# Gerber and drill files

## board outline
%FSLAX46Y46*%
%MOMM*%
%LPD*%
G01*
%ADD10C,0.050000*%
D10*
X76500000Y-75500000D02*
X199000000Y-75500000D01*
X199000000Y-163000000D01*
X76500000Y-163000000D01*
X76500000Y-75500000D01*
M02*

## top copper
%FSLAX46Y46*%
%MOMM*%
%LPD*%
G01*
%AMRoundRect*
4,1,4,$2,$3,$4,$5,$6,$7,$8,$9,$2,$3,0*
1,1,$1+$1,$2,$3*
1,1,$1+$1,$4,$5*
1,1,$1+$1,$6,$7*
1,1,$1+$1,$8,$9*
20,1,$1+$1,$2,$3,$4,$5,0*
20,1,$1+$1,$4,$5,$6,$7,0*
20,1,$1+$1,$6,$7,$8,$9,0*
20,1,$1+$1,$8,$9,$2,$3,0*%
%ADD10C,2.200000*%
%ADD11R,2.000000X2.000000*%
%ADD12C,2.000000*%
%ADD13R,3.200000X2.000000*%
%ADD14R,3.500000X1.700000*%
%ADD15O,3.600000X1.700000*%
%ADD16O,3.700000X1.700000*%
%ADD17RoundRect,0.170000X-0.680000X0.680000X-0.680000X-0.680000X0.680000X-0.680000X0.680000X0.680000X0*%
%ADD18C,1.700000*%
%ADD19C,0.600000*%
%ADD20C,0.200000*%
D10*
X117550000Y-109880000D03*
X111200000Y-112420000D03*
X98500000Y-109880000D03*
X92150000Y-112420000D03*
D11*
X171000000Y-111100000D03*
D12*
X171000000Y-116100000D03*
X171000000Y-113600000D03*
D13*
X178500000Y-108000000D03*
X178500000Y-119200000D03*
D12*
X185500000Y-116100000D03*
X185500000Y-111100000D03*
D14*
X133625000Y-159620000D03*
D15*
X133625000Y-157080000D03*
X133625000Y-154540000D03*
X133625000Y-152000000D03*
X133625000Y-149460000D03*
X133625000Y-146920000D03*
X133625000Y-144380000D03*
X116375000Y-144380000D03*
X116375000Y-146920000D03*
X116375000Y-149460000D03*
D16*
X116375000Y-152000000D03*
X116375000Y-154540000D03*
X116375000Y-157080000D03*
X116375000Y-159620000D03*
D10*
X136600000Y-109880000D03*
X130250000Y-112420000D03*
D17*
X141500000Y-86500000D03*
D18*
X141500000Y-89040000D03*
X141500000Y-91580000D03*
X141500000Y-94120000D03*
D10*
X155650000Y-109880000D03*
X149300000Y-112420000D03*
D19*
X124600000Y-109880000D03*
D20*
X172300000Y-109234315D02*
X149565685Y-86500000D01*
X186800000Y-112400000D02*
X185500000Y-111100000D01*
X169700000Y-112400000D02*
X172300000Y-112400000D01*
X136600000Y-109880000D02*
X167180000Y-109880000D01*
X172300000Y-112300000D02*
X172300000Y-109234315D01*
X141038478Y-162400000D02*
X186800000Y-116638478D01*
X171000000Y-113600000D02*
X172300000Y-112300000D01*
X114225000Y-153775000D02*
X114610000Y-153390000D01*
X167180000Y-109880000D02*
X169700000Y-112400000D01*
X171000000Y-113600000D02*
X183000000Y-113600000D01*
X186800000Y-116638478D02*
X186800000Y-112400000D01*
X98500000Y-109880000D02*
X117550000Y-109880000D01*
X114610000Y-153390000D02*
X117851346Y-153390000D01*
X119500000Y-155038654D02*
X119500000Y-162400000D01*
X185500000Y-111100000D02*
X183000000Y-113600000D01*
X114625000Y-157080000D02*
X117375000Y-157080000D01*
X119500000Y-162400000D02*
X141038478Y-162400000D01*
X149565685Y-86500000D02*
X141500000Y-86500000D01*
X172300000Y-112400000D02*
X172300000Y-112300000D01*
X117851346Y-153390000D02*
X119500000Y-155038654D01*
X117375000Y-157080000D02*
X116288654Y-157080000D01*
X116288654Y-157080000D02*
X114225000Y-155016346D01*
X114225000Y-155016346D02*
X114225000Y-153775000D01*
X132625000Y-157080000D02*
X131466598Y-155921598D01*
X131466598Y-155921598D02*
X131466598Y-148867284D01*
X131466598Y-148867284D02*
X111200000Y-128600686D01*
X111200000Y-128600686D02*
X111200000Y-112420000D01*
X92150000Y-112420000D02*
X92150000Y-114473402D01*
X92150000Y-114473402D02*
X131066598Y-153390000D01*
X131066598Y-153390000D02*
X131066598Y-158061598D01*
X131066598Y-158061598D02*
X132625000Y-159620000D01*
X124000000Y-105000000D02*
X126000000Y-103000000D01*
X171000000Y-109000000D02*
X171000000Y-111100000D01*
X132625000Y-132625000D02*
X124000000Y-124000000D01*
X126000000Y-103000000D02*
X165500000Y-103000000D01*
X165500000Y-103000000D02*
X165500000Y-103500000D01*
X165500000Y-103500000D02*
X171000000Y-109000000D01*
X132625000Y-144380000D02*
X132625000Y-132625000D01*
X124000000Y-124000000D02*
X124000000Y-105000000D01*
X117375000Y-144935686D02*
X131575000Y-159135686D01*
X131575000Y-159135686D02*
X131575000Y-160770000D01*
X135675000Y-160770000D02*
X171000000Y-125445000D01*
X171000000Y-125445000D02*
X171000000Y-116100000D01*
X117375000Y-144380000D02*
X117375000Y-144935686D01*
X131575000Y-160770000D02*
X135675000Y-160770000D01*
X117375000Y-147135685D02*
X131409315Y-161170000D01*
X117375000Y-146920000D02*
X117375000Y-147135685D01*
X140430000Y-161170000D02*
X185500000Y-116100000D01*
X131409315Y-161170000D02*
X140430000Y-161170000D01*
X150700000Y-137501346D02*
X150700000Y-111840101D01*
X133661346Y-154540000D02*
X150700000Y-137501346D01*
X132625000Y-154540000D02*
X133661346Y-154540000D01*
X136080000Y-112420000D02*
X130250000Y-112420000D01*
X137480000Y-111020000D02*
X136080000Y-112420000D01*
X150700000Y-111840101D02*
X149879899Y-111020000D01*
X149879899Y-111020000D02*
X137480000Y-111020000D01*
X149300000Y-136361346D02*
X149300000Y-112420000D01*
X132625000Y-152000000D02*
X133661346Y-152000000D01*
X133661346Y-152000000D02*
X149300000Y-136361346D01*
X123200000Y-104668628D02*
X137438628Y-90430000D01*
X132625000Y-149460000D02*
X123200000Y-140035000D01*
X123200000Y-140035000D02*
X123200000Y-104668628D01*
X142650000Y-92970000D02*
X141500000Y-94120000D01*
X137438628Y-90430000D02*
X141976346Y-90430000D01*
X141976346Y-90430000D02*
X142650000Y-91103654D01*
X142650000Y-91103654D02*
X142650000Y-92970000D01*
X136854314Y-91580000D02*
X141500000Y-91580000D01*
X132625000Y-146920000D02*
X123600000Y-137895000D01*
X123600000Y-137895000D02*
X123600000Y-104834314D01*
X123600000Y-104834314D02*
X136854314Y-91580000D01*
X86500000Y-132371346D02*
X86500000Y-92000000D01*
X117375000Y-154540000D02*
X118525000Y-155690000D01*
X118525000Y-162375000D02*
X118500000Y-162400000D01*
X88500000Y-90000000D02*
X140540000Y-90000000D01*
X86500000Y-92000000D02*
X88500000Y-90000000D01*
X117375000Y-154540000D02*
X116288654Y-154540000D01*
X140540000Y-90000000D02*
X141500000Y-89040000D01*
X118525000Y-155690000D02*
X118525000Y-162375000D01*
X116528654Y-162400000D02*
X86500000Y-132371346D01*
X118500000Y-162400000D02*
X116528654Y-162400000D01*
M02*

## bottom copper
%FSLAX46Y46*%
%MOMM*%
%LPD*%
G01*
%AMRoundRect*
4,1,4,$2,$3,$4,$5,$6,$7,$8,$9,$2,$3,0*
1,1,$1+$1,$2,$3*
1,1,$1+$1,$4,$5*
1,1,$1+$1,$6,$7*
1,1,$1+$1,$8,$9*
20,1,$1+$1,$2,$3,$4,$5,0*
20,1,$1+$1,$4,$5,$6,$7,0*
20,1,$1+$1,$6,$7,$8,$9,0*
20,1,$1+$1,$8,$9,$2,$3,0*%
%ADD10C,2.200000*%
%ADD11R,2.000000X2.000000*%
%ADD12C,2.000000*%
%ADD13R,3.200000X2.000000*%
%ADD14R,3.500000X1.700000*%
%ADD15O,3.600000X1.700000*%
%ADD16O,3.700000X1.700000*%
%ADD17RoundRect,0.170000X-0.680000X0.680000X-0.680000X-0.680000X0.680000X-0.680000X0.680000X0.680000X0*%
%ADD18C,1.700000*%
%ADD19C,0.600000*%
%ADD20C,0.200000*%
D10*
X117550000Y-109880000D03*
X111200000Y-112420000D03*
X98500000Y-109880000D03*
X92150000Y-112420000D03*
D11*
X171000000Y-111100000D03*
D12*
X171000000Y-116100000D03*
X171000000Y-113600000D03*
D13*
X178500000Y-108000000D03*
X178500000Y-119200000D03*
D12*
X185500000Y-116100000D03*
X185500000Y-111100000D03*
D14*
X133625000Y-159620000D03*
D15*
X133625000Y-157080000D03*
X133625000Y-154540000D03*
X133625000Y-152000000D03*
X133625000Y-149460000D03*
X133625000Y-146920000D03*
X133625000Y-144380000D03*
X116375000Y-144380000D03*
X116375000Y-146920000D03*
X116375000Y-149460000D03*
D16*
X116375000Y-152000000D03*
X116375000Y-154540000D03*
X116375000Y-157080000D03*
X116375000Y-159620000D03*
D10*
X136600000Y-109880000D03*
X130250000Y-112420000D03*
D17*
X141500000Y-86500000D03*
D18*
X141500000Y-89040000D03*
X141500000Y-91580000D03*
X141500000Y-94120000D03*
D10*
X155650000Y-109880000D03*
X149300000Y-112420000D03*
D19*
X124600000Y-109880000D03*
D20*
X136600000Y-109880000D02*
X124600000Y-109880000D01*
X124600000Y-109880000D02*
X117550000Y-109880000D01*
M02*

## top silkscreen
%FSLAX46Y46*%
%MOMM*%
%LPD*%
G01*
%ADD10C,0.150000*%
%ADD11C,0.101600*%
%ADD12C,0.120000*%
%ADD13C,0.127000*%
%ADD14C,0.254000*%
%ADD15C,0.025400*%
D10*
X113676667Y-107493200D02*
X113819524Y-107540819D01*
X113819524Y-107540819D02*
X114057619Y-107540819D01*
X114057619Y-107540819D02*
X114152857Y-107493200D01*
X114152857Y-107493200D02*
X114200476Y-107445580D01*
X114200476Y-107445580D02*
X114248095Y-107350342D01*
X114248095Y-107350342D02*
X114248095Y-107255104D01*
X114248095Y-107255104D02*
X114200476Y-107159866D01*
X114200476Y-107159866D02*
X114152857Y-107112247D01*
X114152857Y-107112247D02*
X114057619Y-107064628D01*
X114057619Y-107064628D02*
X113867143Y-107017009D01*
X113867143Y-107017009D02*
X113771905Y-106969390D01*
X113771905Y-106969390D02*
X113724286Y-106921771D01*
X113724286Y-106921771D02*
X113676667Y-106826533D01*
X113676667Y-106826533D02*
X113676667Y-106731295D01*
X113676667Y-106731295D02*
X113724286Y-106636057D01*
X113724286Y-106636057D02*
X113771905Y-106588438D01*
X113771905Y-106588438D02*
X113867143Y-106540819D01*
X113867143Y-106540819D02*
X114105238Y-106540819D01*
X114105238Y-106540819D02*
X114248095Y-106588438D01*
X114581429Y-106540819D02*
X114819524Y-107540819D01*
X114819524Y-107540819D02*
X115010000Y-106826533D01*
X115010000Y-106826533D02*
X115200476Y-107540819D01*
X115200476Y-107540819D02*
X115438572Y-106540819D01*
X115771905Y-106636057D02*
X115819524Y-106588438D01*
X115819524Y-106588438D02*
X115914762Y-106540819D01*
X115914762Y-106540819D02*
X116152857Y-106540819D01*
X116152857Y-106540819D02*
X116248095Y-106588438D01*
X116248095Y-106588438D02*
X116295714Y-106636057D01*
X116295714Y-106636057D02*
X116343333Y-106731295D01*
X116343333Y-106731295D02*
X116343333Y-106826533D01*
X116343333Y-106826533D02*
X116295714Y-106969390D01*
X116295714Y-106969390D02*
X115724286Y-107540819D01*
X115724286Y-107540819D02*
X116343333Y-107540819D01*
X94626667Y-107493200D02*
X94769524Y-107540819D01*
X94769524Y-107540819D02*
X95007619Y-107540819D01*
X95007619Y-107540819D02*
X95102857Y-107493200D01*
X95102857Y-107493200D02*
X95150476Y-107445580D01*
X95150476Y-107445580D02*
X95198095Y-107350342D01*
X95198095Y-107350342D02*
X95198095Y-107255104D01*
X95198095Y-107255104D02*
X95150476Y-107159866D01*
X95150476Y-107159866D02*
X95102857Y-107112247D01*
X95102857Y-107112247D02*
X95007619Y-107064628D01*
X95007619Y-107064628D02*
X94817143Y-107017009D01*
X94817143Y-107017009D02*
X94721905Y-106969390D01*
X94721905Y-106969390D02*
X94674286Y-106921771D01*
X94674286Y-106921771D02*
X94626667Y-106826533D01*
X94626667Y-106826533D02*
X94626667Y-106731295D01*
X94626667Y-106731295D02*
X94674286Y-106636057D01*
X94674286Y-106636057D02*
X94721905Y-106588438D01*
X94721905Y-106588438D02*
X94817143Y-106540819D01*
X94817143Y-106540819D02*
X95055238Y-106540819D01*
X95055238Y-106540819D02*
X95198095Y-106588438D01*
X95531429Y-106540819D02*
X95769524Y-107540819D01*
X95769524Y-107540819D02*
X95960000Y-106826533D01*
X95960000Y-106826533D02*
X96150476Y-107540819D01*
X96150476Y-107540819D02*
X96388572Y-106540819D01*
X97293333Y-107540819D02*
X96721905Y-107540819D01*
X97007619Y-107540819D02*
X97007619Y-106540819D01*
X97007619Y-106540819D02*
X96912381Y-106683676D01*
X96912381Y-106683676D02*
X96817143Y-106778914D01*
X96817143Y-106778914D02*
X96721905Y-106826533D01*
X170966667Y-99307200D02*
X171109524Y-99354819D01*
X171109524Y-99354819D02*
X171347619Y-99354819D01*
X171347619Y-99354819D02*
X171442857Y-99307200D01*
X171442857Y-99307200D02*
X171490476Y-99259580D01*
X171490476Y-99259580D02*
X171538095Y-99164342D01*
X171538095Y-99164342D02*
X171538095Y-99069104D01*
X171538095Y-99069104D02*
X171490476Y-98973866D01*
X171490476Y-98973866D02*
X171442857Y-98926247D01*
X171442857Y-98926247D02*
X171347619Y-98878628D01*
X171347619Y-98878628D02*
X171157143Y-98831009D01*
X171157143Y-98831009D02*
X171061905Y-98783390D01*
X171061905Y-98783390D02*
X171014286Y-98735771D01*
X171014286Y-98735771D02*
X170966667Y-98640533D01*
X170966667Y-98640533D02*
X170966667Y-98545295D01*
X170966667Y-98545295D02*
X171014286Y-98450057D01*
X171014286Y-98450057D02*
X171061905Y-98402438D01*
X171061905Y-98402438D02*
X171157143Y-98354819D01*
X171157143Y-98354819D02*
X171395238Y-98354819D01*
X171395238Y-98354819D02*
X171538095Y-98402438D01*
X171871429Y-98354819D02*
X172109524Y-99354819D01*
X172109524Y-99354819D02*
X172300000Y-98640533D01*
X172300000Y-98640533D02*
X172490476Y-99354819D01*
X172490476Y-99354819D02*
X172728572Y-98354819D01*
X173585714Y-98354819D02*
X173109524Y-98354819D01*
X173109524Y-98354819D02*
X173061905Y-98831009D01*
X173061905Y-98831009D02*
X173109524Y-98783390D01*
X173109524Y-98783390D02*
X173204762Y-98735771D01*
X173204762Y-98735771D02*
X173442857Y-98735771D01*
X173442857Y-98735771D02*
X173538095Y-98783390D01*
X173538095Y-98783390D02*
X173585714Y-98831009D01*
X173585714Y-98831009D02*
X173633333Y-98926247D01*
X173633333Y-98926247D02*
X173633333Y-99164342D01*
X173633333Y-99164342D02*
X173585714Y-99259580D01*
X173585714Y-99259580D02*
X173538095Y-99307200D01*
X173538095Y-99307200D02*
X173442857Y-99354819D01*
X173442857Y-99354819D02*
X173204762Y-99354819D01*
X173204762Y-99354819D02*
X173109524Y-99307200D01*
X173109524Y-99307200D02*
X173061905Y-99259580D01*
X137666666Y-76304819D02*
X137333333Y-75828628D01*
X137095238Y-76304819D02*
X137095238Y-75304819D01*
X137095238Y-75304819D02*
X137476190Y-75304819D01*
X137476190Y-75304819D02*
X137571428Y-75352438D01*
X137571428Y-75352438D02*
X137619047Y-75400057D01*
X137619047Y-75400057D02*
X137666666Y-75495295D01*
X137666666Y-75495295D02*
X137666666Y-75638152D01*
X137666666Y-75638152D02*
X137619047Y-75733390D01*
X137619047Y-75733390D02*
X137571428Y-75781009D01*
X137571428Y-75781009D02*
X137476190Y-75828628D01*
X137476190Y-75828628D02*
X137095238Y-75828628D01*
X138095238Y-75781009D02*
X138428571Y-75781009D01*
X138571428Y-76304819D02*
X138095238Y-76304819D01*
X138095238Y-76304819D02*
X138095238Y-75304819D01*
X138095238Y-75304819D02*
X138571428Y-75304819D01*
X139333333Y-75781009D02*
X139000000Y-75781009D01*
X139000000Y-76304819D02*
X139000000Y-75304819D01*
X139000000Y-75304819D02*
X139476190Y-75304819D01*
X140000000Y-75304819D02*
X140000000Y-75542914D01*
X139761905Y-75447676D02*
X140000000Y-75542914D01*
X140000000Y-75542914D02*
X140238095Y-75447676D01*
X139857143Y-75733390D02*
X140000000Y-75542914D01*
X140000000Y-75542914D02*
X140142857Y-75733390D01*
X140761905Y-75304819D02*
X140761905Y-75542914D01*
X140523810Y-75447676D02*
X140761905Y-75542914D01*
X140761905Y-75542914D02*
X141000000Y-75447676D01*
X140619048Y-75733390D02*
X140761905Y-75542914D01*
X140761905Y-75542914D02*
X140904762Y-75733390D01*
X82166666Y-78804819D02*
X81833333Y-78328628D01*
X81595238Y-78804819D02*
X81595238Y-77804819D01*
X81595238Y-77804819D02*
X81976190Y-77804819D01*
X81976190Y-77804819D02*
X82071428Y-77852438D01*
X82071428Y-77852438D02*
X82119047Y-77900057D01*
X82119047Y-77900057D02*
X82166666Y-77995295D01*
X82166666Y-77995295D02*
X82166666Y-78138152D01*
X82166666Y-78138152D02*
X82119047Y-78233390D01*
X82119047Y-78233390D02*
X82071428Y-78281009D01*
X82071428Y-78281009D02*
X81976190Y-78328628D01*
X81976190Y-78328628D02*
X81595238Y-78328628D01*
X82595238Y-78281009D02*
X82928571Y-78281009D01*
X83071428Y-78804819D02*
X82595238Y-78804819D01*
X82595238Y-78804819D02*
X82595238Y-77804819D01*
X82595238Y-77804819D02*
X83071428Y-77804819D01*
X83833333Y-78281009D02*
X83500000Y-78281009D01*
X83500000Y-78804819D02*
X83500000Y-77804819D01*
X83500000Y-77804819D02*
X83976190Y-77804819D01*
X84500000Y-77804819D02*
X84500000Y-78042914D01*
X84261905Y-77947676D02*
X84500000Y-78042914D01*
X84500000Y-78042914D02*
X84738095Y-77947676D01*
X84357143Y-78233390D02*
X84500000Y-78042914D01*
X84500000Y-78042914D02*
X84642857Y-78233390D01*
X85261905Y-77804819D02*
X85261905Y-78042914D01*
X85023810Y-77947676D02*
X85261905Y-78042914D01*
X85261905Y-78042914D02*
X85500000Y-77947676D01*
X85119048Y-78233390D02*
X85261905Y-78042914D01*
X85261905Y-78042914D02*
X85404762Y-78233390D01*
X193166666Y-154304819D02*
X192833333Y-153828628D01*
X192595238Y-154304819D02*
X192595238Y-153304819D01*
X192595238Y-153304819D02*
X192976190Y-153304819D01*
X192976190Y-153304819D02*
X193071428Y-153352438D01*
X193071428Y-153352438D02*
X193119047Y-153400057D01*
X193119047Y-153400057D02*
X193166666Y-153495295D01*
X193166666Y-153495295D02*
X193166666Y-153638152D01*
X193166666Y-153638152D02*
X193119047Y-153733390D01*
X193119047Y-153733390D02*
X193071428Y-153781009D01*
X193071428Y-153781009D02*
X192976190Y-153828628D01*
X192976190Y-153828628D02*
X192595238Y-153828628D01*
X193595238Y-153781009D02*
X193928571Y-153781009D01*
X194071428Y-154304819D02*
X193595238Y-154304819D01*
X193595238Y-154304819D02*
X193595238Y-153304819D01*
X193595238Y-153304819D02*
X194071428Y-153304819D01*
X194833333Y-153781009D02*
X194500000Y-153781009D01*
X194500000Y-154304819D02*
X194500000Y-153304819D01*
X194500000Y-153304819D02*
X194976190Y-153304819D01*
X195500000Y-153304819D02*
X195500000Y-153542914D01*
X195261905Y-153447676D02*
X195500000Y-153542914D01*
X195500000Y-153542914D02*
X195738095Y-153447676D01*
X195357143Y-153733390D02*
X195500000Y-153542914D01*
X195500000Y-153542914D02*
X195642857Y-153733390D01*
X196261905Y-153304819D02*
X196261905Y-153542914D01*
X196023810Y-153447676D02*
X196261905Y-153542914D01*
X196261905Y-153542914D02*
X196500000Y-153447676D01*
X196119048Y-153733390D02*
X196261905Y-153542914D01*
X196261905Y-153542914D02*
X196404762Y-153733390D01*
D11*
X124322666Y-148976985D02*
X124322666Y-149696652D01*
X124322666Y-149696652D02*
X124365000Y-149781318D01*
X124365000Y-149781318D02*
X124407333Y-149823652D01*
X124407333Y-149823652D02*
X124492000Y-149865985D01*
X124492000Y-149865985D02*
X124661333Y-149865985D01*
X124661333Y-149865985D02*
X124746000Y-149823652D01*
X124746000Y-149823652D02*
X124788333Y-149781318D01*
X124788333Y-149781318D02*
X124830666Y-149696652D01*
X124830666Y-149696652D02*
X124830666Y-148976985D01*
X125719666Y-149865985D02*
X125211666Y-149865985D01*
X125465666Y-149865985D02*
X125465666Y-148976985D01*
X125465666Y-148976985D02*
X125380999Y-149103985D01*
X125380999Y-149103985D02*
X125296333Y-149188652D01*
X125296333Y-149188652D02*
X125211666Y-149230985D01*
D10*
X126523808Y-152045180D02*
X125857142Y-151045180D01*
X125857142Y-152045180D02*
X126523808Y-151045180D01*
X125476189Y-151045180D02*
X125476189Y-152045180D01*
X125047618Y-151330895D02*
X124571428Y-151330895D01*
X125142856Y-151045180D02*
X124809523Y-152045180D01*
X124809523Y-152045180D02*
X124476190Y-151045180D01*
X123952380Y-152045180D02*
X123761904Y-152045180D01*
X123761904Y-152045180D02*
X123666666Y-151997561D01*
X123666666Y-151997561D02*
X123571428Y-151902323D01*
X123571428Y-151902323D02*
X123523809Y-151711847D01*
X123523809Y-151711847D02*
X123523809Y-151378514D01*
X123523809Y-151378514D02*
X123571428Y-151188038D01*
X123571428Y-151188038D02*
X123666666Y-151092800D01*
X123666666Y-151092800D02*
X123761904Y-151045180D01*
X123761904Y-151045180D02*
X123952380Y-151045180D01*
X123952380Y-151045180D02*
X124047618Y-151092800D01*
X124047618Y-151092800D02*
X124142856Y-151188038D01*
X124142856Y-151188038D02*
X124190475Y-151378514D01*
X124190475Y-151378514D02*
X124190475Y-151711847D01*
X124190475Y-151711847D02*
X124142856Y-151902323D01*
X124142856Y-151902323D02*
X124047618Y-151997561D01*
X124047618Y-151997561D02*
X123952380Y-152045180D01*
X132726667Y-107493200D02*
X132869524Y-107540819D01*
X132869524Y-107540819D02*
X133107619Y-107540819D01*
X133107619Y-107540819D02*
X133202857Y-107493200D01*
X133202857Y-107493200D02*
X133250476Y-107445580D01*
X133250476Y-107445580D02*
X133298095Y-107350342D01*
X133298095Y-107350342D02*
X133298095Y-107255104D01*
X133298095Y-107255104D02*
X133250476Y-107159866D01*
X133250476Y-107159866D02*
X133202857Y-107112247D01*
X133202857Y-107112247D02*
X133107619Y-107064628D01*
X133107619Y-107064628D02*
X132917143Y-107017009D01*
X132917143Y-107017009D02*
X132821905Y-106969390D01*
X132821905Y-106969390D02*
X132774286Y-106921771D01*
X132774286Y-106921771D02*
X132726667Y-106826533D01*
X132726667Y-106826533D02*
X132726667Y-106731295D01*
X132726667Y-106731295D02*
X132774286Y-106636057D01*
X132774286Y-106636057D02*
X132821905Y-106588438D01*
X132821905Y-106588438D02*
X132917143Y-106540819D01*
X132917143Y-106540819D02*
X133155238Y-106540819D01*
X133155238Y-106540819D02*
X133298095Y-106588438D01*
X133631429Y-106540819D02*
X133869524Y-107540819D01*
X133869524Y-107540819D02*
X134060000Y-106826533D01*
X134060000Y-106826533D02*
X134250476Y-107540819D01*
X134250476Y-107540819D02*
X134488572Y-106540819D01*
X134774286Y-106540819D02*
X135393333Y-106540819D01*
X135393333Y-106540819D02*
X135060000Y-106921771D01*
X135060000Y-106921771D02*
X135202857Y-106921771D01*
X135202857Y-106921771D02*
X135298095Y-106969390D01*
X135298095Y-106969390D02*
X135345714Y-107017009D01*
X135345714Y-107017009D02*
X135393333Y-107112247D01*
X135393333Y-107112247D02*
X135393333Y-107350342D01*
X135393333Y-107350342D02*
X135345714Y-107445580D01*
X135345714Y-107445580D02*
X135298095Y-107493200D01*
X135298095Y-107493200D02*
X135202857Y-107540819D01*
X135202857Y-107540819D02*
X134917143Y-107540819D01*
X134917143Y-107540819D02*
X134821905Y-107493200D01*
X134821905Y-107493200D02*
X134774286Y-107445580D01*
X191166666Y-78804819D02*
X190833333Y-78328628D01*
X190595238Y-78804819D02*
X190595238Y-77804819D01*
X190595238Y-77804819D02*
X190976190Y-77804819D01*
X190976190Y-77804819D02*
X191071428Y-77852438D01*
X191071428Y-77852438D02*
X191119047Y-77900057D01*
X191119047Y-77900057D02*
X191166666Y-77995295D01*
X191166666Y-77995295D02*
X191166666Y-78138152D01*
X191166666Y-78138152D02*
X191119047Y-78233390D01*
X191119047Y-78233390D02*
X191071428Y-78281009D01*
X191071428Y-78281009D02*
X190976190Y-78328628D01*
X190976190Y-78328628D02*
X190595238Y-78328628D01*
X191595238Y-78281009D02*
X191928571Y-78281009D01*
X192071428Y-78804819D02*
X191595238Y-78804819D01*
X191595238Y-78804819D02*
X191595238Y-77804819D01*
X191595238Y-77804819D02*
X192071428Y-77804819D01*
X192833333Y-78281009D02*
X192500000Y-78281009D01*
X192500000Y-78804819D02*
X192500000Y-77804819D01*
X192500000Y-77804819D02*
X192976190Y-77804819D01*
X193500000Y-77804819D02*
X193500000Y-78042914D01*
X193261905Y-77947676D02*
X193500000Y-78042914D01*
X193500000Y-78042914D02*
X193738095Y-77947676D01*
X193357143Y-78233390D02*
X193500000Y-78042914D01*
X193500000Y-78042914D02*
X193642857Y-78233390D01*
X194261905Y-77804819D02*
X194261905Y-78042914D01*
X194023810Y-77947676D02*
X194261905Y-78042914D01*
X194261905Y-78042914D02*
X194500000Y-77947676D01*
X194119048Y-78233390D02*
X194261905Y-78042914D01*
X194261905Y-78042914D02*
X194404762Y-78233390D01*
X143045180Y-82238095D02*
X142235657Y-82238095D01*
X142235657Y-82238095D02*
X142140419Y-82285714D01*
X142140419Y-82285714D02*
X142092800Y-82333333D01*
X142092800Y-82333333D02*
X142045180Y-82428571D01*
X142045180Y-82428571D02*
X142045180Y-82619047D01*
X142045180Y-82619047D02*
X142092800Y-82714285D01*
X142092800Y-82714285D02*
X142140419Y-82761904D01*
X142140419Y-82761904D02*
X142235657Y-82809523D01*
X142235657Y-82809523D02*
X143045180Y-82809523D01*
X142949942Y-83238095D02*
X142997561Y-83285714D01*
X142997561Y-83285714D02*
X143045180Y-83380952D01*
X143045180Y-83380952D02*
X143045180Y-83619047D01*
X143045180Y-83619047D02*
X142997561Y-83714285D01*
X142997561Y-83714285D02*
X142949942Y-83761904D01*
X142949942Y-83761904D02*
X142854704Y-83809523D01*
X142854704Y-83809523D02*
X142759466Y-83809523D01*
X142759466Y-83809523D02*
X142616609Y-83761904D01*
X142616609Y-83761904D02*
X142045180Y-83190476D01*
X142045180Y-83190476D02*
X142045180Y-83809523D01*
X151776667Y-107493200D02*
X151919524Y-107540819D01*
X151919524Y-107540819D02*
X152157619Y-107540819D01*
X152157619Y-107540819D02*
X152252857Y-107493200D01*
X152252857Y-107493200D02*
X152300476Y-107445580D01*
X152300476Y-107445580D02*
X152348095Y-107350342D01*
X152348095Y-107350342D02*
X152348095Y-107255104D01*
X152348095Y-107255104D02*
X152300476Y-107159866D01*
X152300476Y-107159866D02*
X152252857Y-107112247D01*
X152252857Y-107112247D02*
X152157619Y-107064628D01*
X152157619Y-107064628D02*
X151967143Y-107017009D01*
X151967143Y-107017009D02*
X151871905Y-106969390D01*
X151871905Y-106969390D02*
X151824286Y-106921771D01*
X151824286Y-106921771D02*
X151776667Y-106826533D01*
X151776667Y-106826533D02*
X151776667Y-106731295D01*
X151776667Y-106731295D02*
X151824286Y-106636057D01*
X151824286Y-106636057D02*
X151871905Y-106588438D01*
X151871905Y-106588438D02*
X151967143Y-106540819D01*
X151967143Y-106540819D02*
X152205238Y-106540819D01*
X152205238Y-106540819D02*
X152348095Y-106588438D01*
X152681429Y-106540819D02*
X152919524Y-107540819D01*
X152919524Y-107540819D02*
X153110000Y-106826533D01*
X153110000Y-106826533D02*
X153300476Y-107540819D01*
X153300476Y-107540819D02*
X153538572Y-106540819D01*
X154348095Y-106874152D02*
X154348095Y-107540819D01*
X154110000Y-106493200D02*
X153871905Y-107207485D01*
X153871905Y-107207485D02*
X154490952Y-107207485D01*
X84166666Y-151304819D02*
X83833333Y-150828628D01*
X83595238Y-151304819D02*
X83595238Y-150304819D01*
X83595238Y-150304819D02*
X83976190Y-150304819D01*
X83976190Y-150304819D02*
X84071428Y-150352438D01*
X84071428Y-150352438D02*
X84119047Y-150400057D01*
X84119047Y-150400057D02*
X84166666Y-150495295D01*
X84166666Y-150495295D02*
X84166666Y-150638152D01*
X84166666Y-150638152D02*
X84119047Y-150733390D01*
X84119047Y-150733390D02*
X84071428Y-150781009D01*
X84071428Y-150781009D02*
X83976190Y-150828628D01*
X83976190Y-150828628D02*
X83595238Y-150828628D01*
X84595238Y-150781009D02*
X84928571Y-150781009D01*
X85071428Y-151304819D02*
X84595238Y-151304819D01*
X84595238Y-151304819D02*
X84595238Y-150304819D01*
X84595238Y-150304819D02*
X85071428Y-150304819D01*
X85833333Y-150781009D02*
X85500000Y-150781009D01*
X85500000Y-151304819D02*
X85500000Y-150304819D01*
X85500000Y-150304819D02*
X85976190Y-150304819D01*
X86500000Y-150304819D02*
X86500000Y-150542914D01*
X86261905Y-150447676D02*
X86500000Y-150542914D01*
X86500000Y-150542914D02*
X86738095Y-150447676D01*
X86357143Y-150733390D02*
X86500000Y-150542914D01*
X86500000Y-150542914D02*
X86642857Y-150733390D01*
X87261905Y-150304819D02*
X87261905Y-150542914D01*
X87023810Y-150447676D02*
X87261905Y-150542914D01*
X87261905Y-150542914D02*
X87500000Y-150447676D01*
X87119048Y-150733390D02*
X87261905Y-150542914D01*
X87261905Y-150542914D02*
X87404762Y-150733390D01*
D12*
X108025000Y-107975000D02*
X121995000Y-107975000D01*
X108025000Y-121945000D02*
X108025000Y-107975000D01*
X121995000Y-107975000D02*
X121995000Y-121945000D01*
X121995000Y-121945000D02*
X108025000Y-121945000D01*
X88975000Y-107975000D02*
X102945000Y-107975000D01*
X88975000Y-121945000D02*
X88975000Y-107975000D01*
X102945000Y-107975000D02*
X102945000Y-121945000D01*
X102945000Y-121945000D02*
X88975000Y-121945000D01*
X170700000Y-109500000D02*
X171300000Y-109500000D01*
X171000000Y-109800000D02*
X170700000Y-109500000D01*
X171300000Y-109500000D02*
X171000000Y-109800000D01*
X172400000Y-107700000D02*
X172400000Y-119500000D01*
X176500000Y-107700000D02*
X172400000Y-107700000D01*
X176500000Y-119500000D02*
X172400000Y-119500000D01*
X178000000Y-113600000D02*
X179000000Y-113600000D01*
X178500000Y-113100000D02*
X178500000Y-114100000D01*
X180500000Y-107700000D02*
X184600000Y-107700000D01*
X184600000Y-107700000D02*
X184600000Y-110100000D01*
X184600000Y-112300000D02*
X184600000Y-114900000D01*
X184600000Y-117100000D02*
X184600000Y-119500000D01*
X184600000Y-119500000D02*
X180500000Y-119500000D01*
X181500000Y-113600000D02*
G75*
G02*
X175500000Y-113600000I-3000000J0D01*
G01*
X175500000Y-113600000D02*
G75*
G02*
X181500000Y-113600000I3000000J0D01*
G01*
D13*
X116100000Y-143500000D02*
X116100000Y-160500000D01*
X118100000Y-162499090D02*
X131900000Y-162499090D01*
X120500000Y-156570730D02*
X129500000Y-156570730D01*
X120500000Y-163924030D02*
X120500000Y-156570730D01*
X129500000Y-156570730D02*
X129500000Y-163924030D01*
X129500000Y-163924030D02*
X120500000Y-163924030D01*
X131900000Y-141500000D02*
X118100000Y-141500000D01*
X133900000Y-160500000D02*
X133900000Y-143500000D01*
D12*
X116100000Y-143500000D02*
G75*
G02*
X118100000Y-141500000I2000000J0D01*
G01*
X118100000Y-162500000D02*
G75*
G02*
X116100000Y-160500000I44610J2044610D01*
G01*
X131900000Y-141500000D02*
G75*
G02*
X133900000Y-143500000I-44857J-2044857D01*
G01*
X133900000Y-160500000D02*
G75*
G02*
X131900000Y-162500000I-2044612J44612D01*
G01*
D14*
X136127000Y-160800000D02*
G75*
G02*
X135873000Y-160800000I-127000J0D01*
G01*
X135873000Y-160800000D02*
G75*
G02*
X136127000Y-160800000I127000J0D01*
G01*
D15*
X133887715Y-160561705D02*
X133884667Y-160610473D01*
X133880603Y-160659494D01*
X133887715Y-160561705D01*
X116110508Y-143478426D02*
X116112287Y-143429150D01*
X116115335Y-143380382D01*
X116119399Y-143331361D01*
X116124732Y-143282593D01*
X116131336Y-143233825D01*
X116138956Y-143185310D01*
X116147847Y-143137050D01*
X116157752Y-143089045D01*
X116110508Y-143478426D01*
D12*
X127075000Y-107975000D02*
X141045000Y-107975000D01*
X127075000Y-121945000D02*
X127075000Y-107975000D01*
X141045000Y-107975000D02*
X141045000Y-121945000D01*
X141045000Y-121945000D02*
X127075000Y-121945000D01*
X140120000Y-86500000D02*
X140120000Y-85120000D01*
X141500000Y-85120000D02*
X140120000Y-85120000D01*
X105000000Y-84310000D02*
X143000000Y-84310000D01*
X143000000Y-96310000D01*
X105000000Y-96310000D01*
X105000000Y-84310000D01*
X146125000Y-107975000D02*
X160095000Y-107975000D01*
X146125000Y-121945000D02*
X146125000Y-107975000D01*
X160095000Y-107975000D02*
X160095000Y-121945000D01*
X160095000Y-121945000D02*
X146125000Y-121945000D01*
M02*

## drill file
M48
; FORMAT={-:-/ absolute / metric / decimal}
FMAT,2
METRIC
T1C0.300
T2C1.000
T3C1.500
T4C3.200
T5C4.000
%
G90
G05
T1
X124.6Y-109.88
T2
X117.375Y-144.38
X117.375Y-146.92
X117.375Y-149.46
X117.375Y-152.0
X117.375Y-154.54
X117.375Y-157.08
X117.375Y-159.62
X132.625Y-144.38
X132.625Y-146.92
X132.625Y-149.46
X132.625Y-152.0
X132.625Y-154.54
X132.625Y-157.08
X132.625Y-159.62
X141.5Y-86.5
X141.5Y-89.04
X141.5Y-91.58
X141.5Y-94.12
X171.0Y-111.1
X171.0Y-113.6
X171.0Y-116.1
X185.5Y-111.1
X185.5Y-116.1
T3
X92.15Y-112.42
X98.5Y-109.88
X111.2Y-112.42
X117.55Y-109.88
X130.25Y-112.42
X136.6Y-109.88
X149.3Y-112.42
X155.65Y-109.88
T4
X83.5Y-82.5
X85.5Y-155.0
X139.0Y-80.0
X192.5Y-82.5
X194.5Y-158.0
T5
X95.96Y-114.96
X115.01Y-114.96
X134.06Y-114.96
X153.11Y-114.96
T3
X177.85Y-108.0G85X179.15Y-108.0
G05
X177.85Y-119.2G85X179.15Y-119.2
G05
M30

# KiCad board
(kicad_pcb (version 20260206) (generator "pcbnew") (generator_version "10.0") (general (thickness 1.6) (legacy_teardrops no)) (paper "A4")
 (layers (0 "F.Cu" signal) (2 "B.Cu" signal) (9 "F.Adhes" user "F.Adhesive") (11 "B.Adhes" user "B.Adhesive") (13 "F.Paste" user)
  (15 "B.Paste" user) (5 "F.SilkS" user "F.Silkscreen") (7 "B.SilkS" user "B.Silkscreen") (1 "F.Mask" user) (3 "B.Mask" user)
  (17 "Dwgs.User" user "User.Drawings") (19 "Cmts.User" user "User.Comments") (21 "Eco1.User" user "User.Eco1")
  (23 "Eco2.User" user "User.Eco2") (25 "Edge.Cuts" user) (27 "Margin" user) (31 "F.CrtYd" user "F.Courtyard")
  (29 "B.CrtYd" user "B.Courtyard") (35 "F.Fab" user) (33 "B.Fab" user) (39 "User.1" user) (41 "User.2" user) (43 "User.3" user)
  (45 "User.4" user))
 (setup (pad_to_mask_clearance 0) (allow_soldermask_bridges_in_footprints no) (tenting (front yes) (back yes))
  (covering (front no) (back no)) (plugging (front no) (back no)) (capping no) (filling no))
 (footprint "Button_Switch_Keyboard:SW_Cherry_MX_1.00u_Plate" (layer "F.Cu") (at 117.55 109.88)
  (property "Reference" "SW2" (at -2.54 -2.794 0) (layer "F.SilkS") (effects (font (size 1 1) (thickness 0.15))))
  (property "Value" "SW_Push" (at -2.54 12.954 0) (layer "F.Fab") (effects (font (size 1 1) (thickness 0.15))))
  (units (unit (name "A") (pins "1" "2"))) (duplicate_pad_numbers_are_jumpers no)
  (fp_line (start -9.525 -1.905) (end 4.445 -1.905) (stroke (width 0.12) (type solid)) (layer "F.SilkS"))
  (fp_line (start -9.525 12.065) (end -9.525 -1.905) (stroke (width 0.12) (type solid)) (layer "F.SilkS"))
  (fp_line (start 4.445 -1.905) (end 4.445 12.065) (stroke (width 0.12) (type solid)) (layer "F.SilkS"))
  (fp_line (start 4.445 12.065) (end -9.525 12.065) (stroke (width 0.12) (type solid)) (layer "F.SilkS"))
  (pad "" np_thru_hole circle (at -2.54 5.08) (size 4 4) (drill 4) (layers "*.Cu" "*.Mask"))
  (pad "1" thru_hole circle (at 0 0) (size 2.2 2.2) (drill 1.5) (layers "*.Cu" "*.Mask") (remove_unused_layers no) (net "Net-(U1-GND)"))
  (pad "2" thru_hole circle (at -6.35 2.54) (size 2.2 2.2) (drill 1.5) (layers "*.Cu" "*.Mask") (remove_unused_layers no)
   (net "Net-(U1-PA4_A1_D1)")))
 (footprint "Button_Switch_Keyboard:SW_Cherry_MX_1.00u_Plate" (layer "F.Cu") (at 98.5 109.88)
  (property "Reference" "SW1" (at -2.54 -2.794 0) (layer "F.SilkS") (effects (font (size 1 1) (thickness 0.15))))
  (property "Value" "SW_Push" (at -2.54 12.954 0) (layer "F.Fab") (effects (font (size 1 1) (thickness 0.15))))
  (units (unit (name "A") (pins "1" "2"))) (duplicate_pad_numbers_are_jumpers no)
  (fp_line (start -9.525 -1.905) (end 4.445 -1.905) (stroke (width 0.12) (type solid)) (layer "F.SilkS"))
  (fp_line (start -9.525 12.065) (end -9.525 -1.905) (stroke (width 0.12) (type solid)) (layer "F.SilkS"))
  (fp_line (start 4.445 -1.905) (end 4.445 12.065) (stroke (width 0.12) (type solid)) (layer "F.SilkS"))
  (fp_line (start 4.445 12.065) (end -9.525 12.065) (stroke (width 0.12) (type solid)) (layer "F.SilkS"))
  (pad "" np_thru_hole circle (at -2.54 5.08) (size 4 4) (drill 4) (layers "*.Cu" "*.Mask"))
  (pad "1" thru_hole circle (at 0 0) (size 2.2 2.2) (drill 1.5) (layers "*.Cu" "*.Mask") (remove_unused_layers no) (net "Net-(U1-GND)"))
  (pad "2" thru_hole circle (at -6.35 2.54) (size 2.2 2.2) (drill 1.5) (layers "*.Cu" "*.Mask") (remove_unused_layers no)
   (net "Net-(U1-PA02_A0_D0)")))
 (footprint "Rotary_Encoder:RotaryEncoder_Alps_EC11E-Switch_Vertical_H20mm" (layer "F.Cu") (at 171 111.1)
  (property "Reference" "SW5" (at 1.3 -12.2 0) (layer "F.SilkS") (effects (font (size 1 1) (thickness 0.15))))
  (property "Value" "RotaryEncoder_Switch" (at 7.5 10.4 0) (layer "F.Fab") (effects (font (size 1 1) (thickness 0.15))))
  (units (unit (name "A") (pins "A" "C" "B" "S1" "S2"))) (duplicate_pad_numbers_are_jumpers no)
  (fp_line (start -0.3 -1.6) (end 0.3 -1.6) (stroke (width 0.12) (type solid)) (layer "F.SilkS"))
  (fp_line (start 0 -1.3) (end -0.3 -1.6) (stroke (width 0.12) (type solid)) (layer "F.SilkS"))
  (fp_line (start 0.3 -1.6) (end 0 -1.3) (stroke (width 0.12) (type solid)) (layer "F.SilkS"))
  (fp_line (start 1.4 -3.4) (end 1.4 8.4) (stroke (width 0.12) (type solid)) (layer "F.SilkS"))
  (fp_line (start 5.5 -3.4) (end 1.4 -3.4) (stroke (width 0.12) (type solid)) (layer "F.SilkS"))
  (fp_line (start 5.5 8.4) (end 1.4 8.4) (stroke (width 0.12) (type solid)) (layer "F.SilkS"))
  (fp_line (start 7 2.5) (end 8 2.5) (stroke (width 0.12) (type solid)) (layer "F.SilkS"))
  (fp_line (start 7.5 2) (end 7.5 3) (stroke (width 0.12) (type solid)) (layer "F.SilkS"))
  (fp_line (start 9.5 -3.4) (end 13.6 -3.4) (stroke (width 0.12) (type solid)) (layer "F.SilkS"))
  (fp_line (start 13.6 -3.4) (end 13.6 -1) (stroke (width 0.12) (type solid)) (layer "F.SilkS"))
  (fp_line (start 13.6 1.2) (end 13.6 3.8) (stroke (width 0.12) (type solid)) (layer "F.SilkS"))
  (fp_line (start 13.6 6) (end 13.6 8.4) (stroke (width 0.12) (type solid)) (layer "F.SilkS"))
  (fp_line (start 13.6 8.4) (end 9.5 8.4) (stroke (width 0.12) (type solid)) (layer "F.SilkS"))
  (fp_circle (center 7.5 2.5) (end 10.5 2.5) (stroke (width 0.12) (type solid)) (fill no) (layer "F.SilkS"))
  (pad "A" thru_hole rect (at 0 0) (size 2 2) (drill 1) (layers "*.Cu" "*.Mask") (remove_unused_layers no) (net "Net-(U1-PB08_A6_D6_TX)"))
  (pad "B" thru_hole circle (at 0 5) (size 2 2) (drill 1) (layers "*.Cu" "*.Mask") (remove_unused_layers no) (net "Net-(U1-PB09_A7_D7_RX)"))
  (pad "C" thru_hole circle (at 0 2.5) (size 2 2) (drill 1) (layers "*.Cu" "*.Mask") (remove_unused_layers no) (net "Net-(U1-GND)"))
  (pad "MP" thru_hole rect (at 7.5 -3.1) (size 3.2 2) (drill oval 2.8 1.5) (layers "*.Cu" "*.Mask") (remove_unused_layers no))
  (pad "MP" thru_hole rect (at 7.5 8.1) (size 3.2 2) (drill oval 2.8 1.5) (layers "*.Cu" "*.Mask") (remove_unused_layers no))
  (pad "S1" thru_hole circle (at 14.5 5) (size 2 2) (drill 1) (layers "*.Cu" "*.Mask") (remove_unused_layers no)
   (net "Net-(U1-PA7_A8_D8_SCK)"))
  (pad "S2" thru_hole circle (at 14.5 0) (size 2 2) (drill 1) (layers "*.Cu" "*.Mask") (remove_unused_layers no) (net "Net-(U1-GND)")))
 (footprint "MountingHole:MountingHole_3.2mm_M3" (layer "F.Cu") (at 139 80)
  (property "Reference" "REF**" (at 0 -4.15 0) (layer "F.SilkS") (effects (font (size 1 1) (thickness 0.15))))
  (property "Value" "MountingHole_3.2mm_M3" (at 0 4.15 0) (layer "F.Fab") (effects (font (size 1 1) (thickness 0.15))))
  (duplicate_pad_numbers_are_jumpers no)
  (pad "" np_thru_hole circle (at 0 0) (size 3.2 3.2) (drill 3.2) (layers "*.Cu" "*.Mask")))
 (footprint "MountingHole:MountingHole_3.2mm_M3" (layer "F.Cu") (at 83.5 82.5)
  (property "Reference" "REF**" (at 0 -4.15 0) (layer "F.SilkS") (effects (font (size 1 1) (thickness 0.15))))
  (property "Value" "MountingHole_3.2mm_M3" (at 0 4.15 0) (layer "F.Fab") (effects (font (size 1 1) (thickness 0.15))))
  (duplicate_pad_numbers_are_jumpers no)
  (pad "" np_thru_hole circle (at 0 0) (size 3.2 3.2) (drill 3.2) (layers "*.Cu" "*.Mask")))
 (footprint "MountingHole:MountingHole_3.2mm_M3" (layer "F.Cu") (at 194.5 158)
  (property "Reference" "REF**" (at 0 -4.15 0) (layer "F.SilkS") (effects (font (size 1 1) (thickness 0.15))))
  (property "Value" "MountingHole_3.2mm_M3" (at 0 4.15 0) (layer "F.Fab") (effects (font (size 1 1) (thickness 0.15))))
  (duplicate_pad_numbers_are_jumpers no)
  (pad "" np_thru_hole circle (at 0 0) (size 3.2 3.2) (drill 3.2) (layers "*.Cu" "*.Mask")))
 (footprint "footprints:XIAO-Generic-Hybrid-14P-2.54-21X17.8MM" (layer "F.Cu") (at 125 152 180)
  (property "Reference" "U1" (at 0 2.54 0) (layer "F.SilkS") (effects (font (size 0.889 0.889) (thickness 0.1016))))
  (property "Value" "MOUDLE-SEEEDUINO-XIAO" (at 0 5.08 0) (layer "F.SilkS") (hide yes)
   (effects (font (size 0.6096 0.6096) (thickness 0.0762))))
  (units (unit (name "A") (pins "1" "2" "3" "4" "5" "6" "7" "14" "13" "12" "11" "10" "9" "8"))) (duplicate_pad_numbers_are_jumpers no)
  (fp_line (start 8.9 8.5) (end 8.9 -8.5) (stroke (width 0.127) (type solid)) (layer "F.SilkS"))
  (fp_line (start 6.9 -10.49909) (end -6.9 -10.49909) (stroke (width 0.127) (type solid)) (layer "F.SilkS"))
  (fp_line (start 4.5 -4.57073) (end -4.5 -4.57073) (stroke (width 0.127) (type solid)) (layer "F.SilkS"))
  (fp_line (start 4.5 -11.92403) (end 4.5 -4.57073) (stroke (width 0.127) (type solid)) (layer "F.SilkS"))
  (fp_line (start -4.5 -4.57073) (end -4.5 -11.92403) (stroke (width 0.127) (type solid)) (layer "F.SilkS"))
  (fp_line (start -4.5 -11.92403) (end 4.5 -11.92403) (stroke (width 0.127) (type solid)) (layer "F.SilkS"))
  (fp_line (start -6.9 10.5) (end 6.9 10.5) (stroke (width 0.127) (type solid)) (layer "F.SilkS"))
  (fp_line (start -8.9 -8.5) (end -8.9 8.5) (stroke (width 0.127) (type solid)) (layer "F.SilkS"))
  (fp_arc (start 8.9 8.5) (mid 8.314214 9.914214) (end 6.9 10.5) (stroke (width 0.12) (type solid)) (layer "F.SilkS"))
  (fp_arc (start 6.9 -10.5) (mid 8.301491 -9.901491) (end 8.9 -8.5) (stroke (width 0.12) (type solid)) (layer "F.SilkS"))
  (fp_arc (start -6.9 10.5) (mid -8.301423 9.901423) (end -8.9 8.5) (stroke (width 0.12) (type solid)) (layer "F.SilkS"))
  (fp_arc (start -8.9 -8.5) (mid -8.301491 -9.901491) (end -6.9 -10.5) (stroke (width 0.12) (type solid)) (layer "F.SilkS"))
  (fp_circle (center -11 -8.8) (end -11 -9.054) (stroke (width 0) (type solid)) (fill yes) (layer "F.SilkS"))
  (fp_poly
   (pts (xy -8.887715 -8.561705) (xy -8.884667 -8.610473) (xy -8.880603 -8.659494)) (stroke (width 0.0254) (type solid)) (fill no)
   (layer "F.SilkS"))
  (fp_poly
   (pts (xy 8.889492 8.521574) (xy 8.887713 8.57085) (xy 8.884665 8.619618) (xy 8.880601 8.668639) (xy 8.875268 8.717407)
    (xy 8.868664 8.766175) (xy 8.861044 8.81469) (xy 8.852153 8.86295) (xy 8.842248 8.910955))
   (stroke (width 0.0254) (type solid)) (fill no) (layer "F.SilkS"))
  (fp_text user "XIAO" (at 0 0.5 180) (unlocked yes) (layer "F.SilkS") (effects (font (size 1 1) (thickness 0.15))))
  (pad "1" thru_hole rect (at -7.625 -7.62 180) (size 3.5 1.7) (drill 1 (offset -1 0)) (layers "*.Cu" "*.Mask") (remove_unused_layers no)
   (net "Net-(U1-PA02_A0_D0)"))
  (pad "2" thru_hole oval (at -7.625 -5.08 180) (size 3.6 1.7) (drill 1 (offset -1 0)) (layers "*.Cu" "*.Mask") (remove_unused_layers no)
   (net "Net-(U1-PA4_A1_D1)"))
  (pad "3" thru_hole oval (at -7.625 -2.54 180) (size 3.6 1.7) (drill 1 (offset -1 0)) (layers "*.Cu" "*.Mask") (remove_unused_layers no)
   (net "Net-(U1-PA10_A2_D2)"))
  (pad "4" thru_hole oval (at -7.625 0 180) (size 3.6 1.7) (drill 1 (offset -1 0)) (layers "*.Cu" "*.Mask") (remove_unused_layers no)
   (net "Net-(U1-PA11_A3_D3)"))
  (pad "5" thru_hole oval (at -7.625 2.54 180) (size 3.6 1.7) (drill 1 (offset -1 0)) (layers "*.Cu" "*.Mask") (remove_unused_layers no)
   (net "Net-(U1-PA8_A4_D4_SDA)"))
  (pad "6" thru_hole oval (at -7.625 5.08) (size 3.6 1.7) (drill 1 (offset 1 0)) (layers "*.Cu" "*.Mask") (remove_unused_layers no)
   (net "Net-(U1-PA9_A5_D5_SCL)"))
  (pad "7" thru_hole oval (at -7.625 7.62 180) (size 3.6 1.7) (drill 1 (offset -1 0)) (layers "*.Cu" "*.Mask") (remove_unused_layers no)
   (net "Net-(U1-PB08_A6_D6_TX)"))
  (pad "8" thru_hole oval (at 7.625 7.62 180) (size 3.6 1.7) (drill 1 (offset 1 0)) (layers "*.Cu" "*.Mask") (remove_unused_layers no)
   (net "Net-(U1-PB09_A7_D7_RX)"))
  (pad "9" thru_hole oval (at 7.625 5.08 180) (size 3.6 1.7) (drill 1 (offset 1 0)) (layers "*.Cu" "*.Mask") (remove_unused_layers no)
   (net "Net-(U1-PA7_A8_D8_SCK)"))
  (pad "10" thru_hole oval (at 7.625 2.54 180) (size 3.6 1.7) (drill 1 (offset 1 0)) (layers "*.Cu" "*.Mask") (remove_unused_layers no)
   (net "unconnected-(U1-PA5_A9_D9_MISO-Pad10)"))
  (pad "11" thru_hole oval (at 7.625 0 180) (size 3.7 1.7) (drill 1 (offset 1 0)) (layers "*.Cu" "*.Mask") (remove_unused_layers no)
   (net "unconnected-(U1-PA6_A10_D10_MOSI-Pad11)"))
  (pad "12" thru_hole oval (at 7.625 -2.54 180) (size 3.7 1.7) (drill 1 (offset 1 0)) (layers "*.Cu" "*.Mask") (remove_unused_layers no)
   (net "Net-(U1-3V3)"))
  (pad "13" thru_hole oval (at 7.625 -5.08 180) (size 3.7 1.7) (drill 1 (offset 1 0)) (layers "*.Cu" "*.Mask") (remove_unused_layers no)
   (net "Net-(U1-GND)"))
  (pad "14" thru_hole oval (at 7.625 -7.62 180) (size 3.7 1.7) (drill 1 (offset 1 0)) (layers "*.Cu" "*.Mask") (remove_unused_layers no)
   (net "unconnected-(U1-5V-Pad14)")))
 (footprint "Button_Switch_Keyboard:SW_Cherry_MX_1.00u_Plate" (layer "F.Cu") (at 136.6 109.88)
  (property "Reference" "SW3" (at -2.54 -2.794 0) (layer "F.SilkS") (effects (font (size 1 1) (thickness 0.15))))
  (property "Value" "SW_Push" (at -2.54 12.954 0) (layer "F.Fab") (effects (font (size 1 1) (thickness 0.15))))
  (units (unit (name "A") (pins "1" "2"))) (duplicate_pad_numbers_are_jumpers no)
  (fp_line (start -9.525 -1.905) (end 4.445 -1.905) (stroke (width 0.12) (type solid)) (layer "F.SilkS"))
  (fp_line (start -9.525 12.065) (end -9.525 -1.905) (stroke (width 0.12) (type solid)) (layer "F.SilkS"))
  (fp_line (start 4.445 -1.905) (end 4.445 12.065) (stroke (width 0.12) (type solid)) (layer "F.SilkS"))
  (fp_line (start 4.445 12.065) (end -9.525 12.065) (stroke (width 0.12) (type solid)) (layer "F.SilkS"))
  (pad "" np_thru_hole circle (at -2.54 5.08) (size 4 4) (drill 4) (layers "*.Cu" "*.Mask"))
  (pad "1" thru_hole circle (at 0 0) (size 2.2 2.2) (drill 1.5) (layers "*.Cu" "*.Mask") (remove_unused_layers no) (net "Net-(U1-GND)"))
  (pad "2" thru_hole circle (at -6.35 2.54) (size 2.2 2.2) (drill 1.5) (layers "*.Cu" "*.Mask") (remove_unused_layers no)
   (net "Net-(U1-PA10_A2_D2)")))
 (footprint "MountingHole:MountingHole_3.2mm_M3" (layer "F.Cu") (at 192.5 82.5)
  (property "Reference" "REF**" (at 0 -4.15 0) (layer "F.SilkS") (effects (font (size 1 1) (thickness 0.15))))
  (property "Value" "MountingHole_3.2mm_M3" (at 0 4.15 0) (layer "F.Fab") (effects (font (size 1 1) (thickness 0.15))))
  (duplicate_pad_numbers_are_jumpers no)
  (pad "" np_thru_hole circle (at 0 0) (size 3.2 3.2) (drill 3.2) (layers "*.Cu" "*.Mask")))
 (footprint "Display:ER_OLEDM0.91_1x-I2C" (layer "F.Cu") (at 141.5 86.5 -90)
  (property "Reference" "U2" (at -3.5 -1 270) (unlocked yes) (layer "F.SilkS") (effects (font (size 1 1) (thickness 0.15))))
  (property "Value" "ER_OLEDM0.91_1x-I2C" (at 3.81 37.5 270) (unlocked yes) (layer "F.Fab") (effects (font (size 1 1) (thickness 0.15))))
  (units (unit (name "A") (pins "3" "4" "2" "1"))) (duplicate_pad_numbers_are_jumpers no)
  (fp_line (start 0 1.38) (end -1.38 1.38) (stroke (width 0.12) (type solid)) (layer "F.SilkS"))
  (fp_line (start -1.38 0) (end -1.38 1.38) (stroke (width 0.12) (type solid)) (layer "F.SilkS"))
  (fp_rect (start -2.19 -1.5) (end 9.81 36.5) (stroke (width 0.12) (type solid)) (fill no) (layer "F.SilkS"))
  (pad "1" thru_hole roundrect (at 0 0 270) (size 1.7 1.7) (drill 1) (layers "*.Cu" "*.Mask") (remove_unused_layers no)
   (roundrect_rratio 0.1) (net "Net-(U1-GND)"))
  (pad "2" thru_hole circle (at 2.54 0 270) (size 1.7 1.7) (drill 1) (layers "*.Cu" "*.Mask") (remove_unused_layers no) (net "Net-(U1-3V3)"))
  (pad "3" thru_hole circle (at 5.08 0 270) (size 1.7 1.7) (drill 1) (layers "*.Cu" "*.Mask") (remove_unused_layers no)
   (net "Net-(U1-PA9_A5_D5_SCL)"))
  (pad "4" thru_hole circle (at 7.62 0 270) (size 1.7 1.7) (drill 1) (layers "*.Cu" "*.Mask") (remove_unused_layers no)
   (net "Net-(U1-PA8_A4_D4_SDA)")))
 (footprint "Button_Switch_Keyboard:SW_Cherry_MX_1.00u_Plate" (layer "F.Cu") (at 155.65 109.88)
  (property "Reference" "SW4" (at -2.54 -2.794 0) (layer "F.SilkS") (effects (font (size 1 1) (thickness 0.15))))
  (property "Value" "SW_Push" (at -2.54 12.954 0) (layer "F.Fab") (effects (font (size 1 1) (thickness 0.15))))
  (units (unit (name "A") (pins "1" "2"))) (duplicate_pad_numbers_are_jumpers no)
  (fp_line (start -9.525 -1.905) (end 4.445 -1.905) (stroke (width 0.12) (type solid)) (layer "F.SilkS"))
  (fp_line (start -9.525 12.065) (end -9.525 -1.905) (stroke (width 0.12) (type solid)) (layer "F.SilkS"))
  (fp_line (start 4.445 -1.905) (end 4.445 12.065) (stroke (width 0.12) (type solid)) (layer "F.SilkS"))
  (fp_line (start 4.445 12.065) (end -9.525 12.065) (stroke (width 0.12) (type solid)) (layer "F.SilkS"))
  (pad "" np_thru_hole circle (at -2.54 5.08) (size 4 4) (drill 4) (layers "*.Cu" "*.Mask"))
  (pad "1" thru_hole circle (at 0 0) (size 2.2 2.2) (drill 1.5) (layers "*.Cu" "*.Mask") (remove_unused_layers no) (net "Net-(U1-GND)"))
  (pad "2" thru_hole circle (at -6.35 2.54) (size 2.2 2.2) (drill 1.5) (layers "*.Cu" "*.Mask") (remove_unused_layers no)
   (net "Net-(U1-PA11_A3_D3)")))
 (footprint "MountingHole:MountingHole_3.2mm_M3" (layer "F.Cu") (at 85.5 155)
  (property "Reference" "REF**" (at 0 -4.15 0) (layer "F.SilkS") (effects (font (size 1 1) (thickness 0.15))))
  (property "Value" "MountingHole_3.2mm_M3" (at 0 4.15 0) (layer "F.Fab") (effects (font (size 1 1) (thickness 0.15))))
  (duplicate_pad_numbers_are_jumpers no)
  (pad "" np_thru_hole circle (at 0 0) (size 3.2 3.2) (drill 3.2) (layers "*.Cu" "*.Mask")))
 (gr_rect (start 76.5 75.5) (end 199 163) (stroke (width 0.05) (type default)) (fill no) (layer "Edge.Cuts"))
 (segment (start 172.3 109.234315) (end 149.565685 86.5) (width 0.2) (layer "F.Cu") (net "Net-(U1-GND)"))
 (segment (start 186.8 112.4) (end 185.5 111.1) (width 0.2) (layer "F.Cu") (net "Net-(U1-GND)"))
 (segment (start 169.7 112.4) (end 172.3 112.4) (width 0.2) (layer "F.Cu") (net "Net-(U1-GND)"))
 (segment (start 136.6 109.88) (end 167.18 109.88) (width 0.2) (layer "F.Cu") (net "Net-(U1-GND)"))
 (segment (start 172.3 112.3) (end 172.3 109.234315) (width 0.2) (layer "F.Cu") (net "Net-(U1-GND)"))
 (segment (start 141.038478 162.4) (end 186.8 116.638478) (width 0.2) (layer "F.Cu") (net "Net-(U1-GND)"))
 (segment (start 171 113.6) (end 172.3 112.3) (width 0.2) (layer "F.Cu") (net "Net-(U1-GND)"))
 (segment (start 114.225 153.775) (end 114.61 153.39) (width 0.2) (layer "F.Cu") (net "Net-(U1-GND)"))
 (segment (start 167.18 109.88) (end 169.7 112.4) (width 0.2) (layer "F.Cu") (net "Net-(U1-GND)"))
 (segment (start 171 113.6) (end 183 113.6) (width 0.2) (layer "F.Cu") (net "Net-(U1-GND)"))
 (segment (start 186.8 116.638478) (end 186.8 112.4) (width 0.2) (layer "F.Cu") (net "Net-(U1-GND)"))
 (segment (start 98.5 109.88) (end 117.55 109.88) (width 0.2) (layer "F.Cu") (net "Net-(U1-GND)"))
 (segment (start 114.61 153.39) (end 117.851346 153.39) (width 0.2) (layer "F.Cu") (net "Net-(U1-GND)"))
 (segment (start 119.5 155.038654) (end 119.5 162.4) (width 0.2) (layer "F.Cu") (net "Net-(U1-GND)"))
 (segment (start 185.5 111.1) (end 183 113.6) (width 0.2) (layer "F.Cu") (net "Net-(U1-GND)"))
 (segment (start 114.625 157.08) (end 117.375 157.08) (width 0.2) (layer "F.Cu") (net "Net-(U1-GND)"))
 (segment (start 119.5 162.4) (end 141.038478 162.4) (width 0.2) (layer "F.Cu") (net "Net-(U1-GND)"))
 (segment (start 149.565685 86.5) (end 141.5 86.5) (width 0.2) (layer "F.Cu") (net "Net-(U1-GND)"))
 (segment (start 172.3 112.4) (end 172.3 112.3) (width 0.2) (layer "F.Cu") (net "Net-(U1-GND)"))
 (segment (start 117.851346 153.39) (end 119.5 155.038654) (width 0.2) (layer "F.Cu") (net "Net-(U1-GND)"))
 (segment (start 117.375 157.08) (end 116.288654 157.08) (width 0.2) (layer "F.Cu") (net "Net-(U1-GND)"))
 (segment (start 116.288654 157.08) (end 114.225 155.016346) (width 0.2) (layer "F.Cu") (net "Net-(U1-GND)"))
 (segment (start 114.225 155.016346) (end 114.225 153.775) (width 0.2) (layer "F.Cu") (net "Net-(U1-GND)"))
 (via (at 124.6 109.88) (size 0.6) (drill 0.3) (layers "F.Cu" "B.Cu") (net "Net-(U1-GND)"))
 (segment (start 136.6 109.88) (end 124.6 109.88) (width 0.2) (layer "B.Cu") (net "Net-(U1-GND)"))
 (segment (start 124.6 109.88) (end 117.55 109.88) (width 0.2) (layer "B.Cu") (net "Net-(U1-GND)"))
 (segment (start 132.625 157.08) (end 131.466598 155.921598) (width 0.2) (layer "F.Cu") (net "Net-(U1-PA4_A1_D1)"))
 (segment (start 131.466598 155.921598) (end 131.466598 148.867284) (width 0.2) (layer "F.Cu") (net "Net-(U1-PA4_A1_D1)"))
 (segment (start 131.466598 148.867284) (end 111.2 128.600686) (width 0.2) (layer "F.Cu") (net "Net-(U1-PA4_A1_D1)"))
 (segment (start 111.2 128.600686) (end 111.2 112.42) (width 0.2) (layer "F.Cu") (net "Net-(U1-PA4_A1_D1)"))
 (segment (start 92.15 112.42) (end 92.15 114.473402) (width 0.2) (layer "F.Cu") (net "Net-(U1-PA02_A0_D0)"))
 (segment (start 92.15 114.473402) (end 131.066598 153.39) (width 0.2) (layer "F.Cu") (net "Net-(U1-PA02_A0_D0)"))
 (segment (start 131.066598 153.39) (end 131.066598 158.061598) (width 0.2) (layer "F.Cu") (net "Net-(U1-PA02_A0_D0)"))
 (segment (start 131.066598 158.061598) (end 132.625 159.62) (width 0.2) (layer "F.Cu") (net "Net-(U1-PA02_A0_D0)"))
 (segment (start 124 105) (end 126 103) (width 0.2) (layer "F.Cu") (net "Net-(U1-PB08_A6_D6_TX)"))
 (segment (start 171 109) (end 171 111.1) (width 0.2) (layer "F.Cu") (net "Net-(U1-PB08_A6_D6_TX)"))
 (segment (start 132.625 132.625) (end 124 124) (width 0.2) (layer "F.Cu") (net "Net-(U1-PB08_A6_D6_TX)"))
 (segment (start 126 103) (end 165.5 103) (width 0.2) (layer "F.Cu") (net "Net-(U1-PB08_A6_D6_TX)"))
 (segment (start 165.5 103) (end 165.5 103.5) (width 0.2) (layer "F.Cu") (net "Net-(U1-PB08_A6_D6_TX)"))
 (segment (start 165.5 103.5) (end 171 109) (width 0.2) (layer "F.Cu") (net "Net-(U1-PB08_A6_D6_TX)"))
 (segment (start 132.625 144.38) (end 132.625 132.625) (width 0.2) (layer "F.Cu") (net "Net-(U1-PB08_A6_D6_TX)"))
 (segment (start 124 124) (end 124 105) (width 0.2) (layer "F.Cu") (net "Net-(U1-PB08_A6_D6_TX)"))
 (segment (start 117.375 144.935686) (end 131.575 159.135686) (width 0.2) (layer "F.Cu") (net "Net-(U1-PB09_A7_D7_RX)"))
 (segment (start 131.575 159.135686) (end 131.575 160.77) (width 0.2) (layer "F.Cu") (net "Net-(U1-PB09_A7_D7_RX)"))
 (segment (start 135.675 160.77) (end 171 125.445) (width 0.2) (layer "F.Cu") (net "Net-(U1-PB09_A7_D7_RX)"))
 (segment (start 171 125.445) (end 171 116.1) (width 0.2) (layer "F.Cu") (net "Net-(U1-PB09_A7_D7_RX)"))
 (segment (start 117.375 144.38) (end 117.375 144.935686) (width 0.2) (layer "F.Cu") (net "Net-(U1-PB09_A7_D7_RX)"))
 (segment (start 131.575 160.77) (end 135.675 160.77) (width 0.2) (layer "F.Cu") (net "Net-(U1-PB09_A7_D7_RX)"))
 (segment (start 117.375 147.135685) (end 131.409315 161.17) (width 0.2) (layer "F.Cu") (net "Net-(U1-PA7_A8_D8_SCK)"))
 (segment (start 117.375 146.92) (end 117.375 147.135685) (width 0.2) (layer "F.Cu") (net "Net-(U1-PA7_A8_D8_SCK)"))
 (segment (start 140.43 161.17) (end 185.5 116.1) (width 0.2) (layer "F.Cu") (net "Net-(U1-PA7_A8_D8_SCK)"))
 (segment (start 131.409315 161.17) (end 140.43 161.17) (width 0.2) (layer "F.Cu") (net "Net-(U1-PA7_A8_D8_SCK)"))
 (segment (start 150.7 137.501346) (end 150.7 111.840101) (width 0.2) (layer "F.Cu") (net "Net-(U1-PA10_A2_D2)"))
 (segment (start 133.661346 154.54) (end 150.7 137.501346) (width 0.2) (layer "F.Cu") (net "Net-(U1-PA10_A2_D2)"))
 (segment (start 132.625 154.54) (end 133.661346 154.54) (width 0.2) (layer "F.Cu") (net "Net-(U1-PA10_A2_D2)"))
 (segment (start 136.08 112.42) (end 130.25 112.42) (width 0.2) (layer "F.Cu") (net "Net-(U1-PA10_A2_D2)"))
 (segment (start 137.48 111.02) (end 136.08 112.42) (width 0.2) (layer "F.Cu") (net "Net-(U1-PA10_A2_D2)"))
 (segment (start 150.7 111.840101) (end 149.879899 111.02) (width 0.2) (layer "F.Cu") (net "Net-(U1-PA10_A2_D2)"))
 (segment (start 149.879899 111.02) (end 137.48 111.02) (width 0.2) (layer "F.Cu") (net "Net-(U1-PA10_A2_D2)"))
 (segment (start 149.3 136.361346) (end 149.3 112.42) (width 0.2) (layer "F.Cu") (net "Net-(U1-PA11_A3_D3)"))
 (segment (start 132.625 152) (end 133.661346 152) (width 0.2) (layer "F.Cu") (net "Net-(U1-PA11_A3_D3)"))
 (segment (start 133.661346 152) (end 149.3 136.361346) (width 0.2) (layer "F.Cu") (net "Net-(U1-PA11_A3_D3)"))
 (segment (start 123.2 104.668628) (end 137.438628 90.43) (width 0.2) (layer "F.Cu") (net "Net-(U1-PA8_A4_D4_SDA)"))
 (segment (start 132.625 149.46) (end 123.2 140.035) (width 0.2) (layer "F.Cu") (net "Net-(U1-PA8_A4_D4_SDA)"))
 (segment (start 123.2 140.035) (end 123.2 104.668628) (width 0.2) (layer "F.Cu") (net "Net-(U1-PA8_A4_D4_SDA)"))
 (segment (start 142.65 92.97) (end 141.5 94.12) (width 0.2) (layer "F.Cu") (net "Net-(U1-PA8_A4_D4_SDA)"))
 (segment (start 137.438628 90.43) (end 141.976346 90.43) (width 0.2) (layer "F.Cu") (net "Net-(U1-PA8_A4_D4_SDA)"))
 (segment (start 141.976346 90.43) (end 142.65 91.103654) (width 0.2) (layer "F.Cu") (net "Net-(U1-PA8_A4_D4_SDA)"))
 (segment (start 142.65 91.103654) (end 142.65 92.97) (width 0.2) (layer "F.Cu") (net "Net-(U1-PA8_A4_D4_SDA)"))
 (segment (start 136.854314 91.58) (end 141.5 91.58) (width 0.2) (layer "F.Cu") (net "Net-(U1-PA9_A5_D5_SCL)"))
 (segment (start 132.625 146.92) (end 123.6 137.895) (width 0.2) (layer "F.Cu") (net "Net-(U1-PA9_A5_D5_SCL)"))
 (segment (start 123.6 137.895) (end 123.6 104.834314) (width 0.2) (layer "F.Cu") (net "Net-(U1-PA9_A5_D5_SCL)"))
 (segment (start 123.6 104.834314) (end 136.854314 91.58) (width 0.2) (layer "F.Cu") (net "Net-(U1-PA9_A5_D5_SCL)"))
 (segment (start 86.5 132.371346) (end 86.5 92) (width 0.2) (layer "F.Cu") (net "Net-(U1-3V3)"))
 (segment (start 117.375 154.54) (end 118.525 155.69) (width 0.2) (layer "F.Cu") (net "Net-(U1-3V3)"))
 (segment (start 118.525 162.375) (end 118.5 162.4) (width 0.2) (layer "F.Cu") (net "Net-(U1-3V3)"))
 (segment (start 88.5 90) (end 140.54 90) (width 0.2) (layer "F.Cu") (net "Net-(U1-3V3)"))
 (segment (start 86.5 92) (end 88.5 90) (width 0.2) (layer "F.Cu") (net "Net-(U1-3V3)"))
 (segment (start 117.375 154.54) (end 116.288654 154.54) (width 0.2) (layer "F.Cu") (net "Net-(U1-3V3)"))
 (segment (start 140.54 90) (end 141.5 89.04) (width 0.2) (layer "F.Cu") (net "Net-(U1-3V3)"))
 (segment (start 118.525 155.69) (end 118.525 162.375) (width 0.2) (layer "F.Cu") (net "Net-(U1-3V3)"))
 (segment (start 116.528654 162.4) (end 86.5 132.371346) (width 0.2) (layer "F.Cu") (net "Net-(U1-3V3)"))
 (segment (start 118.5 162.4) (end 116.528654 162.4) (width 0.2) (layer "F.Cu") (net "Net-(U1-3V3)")))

